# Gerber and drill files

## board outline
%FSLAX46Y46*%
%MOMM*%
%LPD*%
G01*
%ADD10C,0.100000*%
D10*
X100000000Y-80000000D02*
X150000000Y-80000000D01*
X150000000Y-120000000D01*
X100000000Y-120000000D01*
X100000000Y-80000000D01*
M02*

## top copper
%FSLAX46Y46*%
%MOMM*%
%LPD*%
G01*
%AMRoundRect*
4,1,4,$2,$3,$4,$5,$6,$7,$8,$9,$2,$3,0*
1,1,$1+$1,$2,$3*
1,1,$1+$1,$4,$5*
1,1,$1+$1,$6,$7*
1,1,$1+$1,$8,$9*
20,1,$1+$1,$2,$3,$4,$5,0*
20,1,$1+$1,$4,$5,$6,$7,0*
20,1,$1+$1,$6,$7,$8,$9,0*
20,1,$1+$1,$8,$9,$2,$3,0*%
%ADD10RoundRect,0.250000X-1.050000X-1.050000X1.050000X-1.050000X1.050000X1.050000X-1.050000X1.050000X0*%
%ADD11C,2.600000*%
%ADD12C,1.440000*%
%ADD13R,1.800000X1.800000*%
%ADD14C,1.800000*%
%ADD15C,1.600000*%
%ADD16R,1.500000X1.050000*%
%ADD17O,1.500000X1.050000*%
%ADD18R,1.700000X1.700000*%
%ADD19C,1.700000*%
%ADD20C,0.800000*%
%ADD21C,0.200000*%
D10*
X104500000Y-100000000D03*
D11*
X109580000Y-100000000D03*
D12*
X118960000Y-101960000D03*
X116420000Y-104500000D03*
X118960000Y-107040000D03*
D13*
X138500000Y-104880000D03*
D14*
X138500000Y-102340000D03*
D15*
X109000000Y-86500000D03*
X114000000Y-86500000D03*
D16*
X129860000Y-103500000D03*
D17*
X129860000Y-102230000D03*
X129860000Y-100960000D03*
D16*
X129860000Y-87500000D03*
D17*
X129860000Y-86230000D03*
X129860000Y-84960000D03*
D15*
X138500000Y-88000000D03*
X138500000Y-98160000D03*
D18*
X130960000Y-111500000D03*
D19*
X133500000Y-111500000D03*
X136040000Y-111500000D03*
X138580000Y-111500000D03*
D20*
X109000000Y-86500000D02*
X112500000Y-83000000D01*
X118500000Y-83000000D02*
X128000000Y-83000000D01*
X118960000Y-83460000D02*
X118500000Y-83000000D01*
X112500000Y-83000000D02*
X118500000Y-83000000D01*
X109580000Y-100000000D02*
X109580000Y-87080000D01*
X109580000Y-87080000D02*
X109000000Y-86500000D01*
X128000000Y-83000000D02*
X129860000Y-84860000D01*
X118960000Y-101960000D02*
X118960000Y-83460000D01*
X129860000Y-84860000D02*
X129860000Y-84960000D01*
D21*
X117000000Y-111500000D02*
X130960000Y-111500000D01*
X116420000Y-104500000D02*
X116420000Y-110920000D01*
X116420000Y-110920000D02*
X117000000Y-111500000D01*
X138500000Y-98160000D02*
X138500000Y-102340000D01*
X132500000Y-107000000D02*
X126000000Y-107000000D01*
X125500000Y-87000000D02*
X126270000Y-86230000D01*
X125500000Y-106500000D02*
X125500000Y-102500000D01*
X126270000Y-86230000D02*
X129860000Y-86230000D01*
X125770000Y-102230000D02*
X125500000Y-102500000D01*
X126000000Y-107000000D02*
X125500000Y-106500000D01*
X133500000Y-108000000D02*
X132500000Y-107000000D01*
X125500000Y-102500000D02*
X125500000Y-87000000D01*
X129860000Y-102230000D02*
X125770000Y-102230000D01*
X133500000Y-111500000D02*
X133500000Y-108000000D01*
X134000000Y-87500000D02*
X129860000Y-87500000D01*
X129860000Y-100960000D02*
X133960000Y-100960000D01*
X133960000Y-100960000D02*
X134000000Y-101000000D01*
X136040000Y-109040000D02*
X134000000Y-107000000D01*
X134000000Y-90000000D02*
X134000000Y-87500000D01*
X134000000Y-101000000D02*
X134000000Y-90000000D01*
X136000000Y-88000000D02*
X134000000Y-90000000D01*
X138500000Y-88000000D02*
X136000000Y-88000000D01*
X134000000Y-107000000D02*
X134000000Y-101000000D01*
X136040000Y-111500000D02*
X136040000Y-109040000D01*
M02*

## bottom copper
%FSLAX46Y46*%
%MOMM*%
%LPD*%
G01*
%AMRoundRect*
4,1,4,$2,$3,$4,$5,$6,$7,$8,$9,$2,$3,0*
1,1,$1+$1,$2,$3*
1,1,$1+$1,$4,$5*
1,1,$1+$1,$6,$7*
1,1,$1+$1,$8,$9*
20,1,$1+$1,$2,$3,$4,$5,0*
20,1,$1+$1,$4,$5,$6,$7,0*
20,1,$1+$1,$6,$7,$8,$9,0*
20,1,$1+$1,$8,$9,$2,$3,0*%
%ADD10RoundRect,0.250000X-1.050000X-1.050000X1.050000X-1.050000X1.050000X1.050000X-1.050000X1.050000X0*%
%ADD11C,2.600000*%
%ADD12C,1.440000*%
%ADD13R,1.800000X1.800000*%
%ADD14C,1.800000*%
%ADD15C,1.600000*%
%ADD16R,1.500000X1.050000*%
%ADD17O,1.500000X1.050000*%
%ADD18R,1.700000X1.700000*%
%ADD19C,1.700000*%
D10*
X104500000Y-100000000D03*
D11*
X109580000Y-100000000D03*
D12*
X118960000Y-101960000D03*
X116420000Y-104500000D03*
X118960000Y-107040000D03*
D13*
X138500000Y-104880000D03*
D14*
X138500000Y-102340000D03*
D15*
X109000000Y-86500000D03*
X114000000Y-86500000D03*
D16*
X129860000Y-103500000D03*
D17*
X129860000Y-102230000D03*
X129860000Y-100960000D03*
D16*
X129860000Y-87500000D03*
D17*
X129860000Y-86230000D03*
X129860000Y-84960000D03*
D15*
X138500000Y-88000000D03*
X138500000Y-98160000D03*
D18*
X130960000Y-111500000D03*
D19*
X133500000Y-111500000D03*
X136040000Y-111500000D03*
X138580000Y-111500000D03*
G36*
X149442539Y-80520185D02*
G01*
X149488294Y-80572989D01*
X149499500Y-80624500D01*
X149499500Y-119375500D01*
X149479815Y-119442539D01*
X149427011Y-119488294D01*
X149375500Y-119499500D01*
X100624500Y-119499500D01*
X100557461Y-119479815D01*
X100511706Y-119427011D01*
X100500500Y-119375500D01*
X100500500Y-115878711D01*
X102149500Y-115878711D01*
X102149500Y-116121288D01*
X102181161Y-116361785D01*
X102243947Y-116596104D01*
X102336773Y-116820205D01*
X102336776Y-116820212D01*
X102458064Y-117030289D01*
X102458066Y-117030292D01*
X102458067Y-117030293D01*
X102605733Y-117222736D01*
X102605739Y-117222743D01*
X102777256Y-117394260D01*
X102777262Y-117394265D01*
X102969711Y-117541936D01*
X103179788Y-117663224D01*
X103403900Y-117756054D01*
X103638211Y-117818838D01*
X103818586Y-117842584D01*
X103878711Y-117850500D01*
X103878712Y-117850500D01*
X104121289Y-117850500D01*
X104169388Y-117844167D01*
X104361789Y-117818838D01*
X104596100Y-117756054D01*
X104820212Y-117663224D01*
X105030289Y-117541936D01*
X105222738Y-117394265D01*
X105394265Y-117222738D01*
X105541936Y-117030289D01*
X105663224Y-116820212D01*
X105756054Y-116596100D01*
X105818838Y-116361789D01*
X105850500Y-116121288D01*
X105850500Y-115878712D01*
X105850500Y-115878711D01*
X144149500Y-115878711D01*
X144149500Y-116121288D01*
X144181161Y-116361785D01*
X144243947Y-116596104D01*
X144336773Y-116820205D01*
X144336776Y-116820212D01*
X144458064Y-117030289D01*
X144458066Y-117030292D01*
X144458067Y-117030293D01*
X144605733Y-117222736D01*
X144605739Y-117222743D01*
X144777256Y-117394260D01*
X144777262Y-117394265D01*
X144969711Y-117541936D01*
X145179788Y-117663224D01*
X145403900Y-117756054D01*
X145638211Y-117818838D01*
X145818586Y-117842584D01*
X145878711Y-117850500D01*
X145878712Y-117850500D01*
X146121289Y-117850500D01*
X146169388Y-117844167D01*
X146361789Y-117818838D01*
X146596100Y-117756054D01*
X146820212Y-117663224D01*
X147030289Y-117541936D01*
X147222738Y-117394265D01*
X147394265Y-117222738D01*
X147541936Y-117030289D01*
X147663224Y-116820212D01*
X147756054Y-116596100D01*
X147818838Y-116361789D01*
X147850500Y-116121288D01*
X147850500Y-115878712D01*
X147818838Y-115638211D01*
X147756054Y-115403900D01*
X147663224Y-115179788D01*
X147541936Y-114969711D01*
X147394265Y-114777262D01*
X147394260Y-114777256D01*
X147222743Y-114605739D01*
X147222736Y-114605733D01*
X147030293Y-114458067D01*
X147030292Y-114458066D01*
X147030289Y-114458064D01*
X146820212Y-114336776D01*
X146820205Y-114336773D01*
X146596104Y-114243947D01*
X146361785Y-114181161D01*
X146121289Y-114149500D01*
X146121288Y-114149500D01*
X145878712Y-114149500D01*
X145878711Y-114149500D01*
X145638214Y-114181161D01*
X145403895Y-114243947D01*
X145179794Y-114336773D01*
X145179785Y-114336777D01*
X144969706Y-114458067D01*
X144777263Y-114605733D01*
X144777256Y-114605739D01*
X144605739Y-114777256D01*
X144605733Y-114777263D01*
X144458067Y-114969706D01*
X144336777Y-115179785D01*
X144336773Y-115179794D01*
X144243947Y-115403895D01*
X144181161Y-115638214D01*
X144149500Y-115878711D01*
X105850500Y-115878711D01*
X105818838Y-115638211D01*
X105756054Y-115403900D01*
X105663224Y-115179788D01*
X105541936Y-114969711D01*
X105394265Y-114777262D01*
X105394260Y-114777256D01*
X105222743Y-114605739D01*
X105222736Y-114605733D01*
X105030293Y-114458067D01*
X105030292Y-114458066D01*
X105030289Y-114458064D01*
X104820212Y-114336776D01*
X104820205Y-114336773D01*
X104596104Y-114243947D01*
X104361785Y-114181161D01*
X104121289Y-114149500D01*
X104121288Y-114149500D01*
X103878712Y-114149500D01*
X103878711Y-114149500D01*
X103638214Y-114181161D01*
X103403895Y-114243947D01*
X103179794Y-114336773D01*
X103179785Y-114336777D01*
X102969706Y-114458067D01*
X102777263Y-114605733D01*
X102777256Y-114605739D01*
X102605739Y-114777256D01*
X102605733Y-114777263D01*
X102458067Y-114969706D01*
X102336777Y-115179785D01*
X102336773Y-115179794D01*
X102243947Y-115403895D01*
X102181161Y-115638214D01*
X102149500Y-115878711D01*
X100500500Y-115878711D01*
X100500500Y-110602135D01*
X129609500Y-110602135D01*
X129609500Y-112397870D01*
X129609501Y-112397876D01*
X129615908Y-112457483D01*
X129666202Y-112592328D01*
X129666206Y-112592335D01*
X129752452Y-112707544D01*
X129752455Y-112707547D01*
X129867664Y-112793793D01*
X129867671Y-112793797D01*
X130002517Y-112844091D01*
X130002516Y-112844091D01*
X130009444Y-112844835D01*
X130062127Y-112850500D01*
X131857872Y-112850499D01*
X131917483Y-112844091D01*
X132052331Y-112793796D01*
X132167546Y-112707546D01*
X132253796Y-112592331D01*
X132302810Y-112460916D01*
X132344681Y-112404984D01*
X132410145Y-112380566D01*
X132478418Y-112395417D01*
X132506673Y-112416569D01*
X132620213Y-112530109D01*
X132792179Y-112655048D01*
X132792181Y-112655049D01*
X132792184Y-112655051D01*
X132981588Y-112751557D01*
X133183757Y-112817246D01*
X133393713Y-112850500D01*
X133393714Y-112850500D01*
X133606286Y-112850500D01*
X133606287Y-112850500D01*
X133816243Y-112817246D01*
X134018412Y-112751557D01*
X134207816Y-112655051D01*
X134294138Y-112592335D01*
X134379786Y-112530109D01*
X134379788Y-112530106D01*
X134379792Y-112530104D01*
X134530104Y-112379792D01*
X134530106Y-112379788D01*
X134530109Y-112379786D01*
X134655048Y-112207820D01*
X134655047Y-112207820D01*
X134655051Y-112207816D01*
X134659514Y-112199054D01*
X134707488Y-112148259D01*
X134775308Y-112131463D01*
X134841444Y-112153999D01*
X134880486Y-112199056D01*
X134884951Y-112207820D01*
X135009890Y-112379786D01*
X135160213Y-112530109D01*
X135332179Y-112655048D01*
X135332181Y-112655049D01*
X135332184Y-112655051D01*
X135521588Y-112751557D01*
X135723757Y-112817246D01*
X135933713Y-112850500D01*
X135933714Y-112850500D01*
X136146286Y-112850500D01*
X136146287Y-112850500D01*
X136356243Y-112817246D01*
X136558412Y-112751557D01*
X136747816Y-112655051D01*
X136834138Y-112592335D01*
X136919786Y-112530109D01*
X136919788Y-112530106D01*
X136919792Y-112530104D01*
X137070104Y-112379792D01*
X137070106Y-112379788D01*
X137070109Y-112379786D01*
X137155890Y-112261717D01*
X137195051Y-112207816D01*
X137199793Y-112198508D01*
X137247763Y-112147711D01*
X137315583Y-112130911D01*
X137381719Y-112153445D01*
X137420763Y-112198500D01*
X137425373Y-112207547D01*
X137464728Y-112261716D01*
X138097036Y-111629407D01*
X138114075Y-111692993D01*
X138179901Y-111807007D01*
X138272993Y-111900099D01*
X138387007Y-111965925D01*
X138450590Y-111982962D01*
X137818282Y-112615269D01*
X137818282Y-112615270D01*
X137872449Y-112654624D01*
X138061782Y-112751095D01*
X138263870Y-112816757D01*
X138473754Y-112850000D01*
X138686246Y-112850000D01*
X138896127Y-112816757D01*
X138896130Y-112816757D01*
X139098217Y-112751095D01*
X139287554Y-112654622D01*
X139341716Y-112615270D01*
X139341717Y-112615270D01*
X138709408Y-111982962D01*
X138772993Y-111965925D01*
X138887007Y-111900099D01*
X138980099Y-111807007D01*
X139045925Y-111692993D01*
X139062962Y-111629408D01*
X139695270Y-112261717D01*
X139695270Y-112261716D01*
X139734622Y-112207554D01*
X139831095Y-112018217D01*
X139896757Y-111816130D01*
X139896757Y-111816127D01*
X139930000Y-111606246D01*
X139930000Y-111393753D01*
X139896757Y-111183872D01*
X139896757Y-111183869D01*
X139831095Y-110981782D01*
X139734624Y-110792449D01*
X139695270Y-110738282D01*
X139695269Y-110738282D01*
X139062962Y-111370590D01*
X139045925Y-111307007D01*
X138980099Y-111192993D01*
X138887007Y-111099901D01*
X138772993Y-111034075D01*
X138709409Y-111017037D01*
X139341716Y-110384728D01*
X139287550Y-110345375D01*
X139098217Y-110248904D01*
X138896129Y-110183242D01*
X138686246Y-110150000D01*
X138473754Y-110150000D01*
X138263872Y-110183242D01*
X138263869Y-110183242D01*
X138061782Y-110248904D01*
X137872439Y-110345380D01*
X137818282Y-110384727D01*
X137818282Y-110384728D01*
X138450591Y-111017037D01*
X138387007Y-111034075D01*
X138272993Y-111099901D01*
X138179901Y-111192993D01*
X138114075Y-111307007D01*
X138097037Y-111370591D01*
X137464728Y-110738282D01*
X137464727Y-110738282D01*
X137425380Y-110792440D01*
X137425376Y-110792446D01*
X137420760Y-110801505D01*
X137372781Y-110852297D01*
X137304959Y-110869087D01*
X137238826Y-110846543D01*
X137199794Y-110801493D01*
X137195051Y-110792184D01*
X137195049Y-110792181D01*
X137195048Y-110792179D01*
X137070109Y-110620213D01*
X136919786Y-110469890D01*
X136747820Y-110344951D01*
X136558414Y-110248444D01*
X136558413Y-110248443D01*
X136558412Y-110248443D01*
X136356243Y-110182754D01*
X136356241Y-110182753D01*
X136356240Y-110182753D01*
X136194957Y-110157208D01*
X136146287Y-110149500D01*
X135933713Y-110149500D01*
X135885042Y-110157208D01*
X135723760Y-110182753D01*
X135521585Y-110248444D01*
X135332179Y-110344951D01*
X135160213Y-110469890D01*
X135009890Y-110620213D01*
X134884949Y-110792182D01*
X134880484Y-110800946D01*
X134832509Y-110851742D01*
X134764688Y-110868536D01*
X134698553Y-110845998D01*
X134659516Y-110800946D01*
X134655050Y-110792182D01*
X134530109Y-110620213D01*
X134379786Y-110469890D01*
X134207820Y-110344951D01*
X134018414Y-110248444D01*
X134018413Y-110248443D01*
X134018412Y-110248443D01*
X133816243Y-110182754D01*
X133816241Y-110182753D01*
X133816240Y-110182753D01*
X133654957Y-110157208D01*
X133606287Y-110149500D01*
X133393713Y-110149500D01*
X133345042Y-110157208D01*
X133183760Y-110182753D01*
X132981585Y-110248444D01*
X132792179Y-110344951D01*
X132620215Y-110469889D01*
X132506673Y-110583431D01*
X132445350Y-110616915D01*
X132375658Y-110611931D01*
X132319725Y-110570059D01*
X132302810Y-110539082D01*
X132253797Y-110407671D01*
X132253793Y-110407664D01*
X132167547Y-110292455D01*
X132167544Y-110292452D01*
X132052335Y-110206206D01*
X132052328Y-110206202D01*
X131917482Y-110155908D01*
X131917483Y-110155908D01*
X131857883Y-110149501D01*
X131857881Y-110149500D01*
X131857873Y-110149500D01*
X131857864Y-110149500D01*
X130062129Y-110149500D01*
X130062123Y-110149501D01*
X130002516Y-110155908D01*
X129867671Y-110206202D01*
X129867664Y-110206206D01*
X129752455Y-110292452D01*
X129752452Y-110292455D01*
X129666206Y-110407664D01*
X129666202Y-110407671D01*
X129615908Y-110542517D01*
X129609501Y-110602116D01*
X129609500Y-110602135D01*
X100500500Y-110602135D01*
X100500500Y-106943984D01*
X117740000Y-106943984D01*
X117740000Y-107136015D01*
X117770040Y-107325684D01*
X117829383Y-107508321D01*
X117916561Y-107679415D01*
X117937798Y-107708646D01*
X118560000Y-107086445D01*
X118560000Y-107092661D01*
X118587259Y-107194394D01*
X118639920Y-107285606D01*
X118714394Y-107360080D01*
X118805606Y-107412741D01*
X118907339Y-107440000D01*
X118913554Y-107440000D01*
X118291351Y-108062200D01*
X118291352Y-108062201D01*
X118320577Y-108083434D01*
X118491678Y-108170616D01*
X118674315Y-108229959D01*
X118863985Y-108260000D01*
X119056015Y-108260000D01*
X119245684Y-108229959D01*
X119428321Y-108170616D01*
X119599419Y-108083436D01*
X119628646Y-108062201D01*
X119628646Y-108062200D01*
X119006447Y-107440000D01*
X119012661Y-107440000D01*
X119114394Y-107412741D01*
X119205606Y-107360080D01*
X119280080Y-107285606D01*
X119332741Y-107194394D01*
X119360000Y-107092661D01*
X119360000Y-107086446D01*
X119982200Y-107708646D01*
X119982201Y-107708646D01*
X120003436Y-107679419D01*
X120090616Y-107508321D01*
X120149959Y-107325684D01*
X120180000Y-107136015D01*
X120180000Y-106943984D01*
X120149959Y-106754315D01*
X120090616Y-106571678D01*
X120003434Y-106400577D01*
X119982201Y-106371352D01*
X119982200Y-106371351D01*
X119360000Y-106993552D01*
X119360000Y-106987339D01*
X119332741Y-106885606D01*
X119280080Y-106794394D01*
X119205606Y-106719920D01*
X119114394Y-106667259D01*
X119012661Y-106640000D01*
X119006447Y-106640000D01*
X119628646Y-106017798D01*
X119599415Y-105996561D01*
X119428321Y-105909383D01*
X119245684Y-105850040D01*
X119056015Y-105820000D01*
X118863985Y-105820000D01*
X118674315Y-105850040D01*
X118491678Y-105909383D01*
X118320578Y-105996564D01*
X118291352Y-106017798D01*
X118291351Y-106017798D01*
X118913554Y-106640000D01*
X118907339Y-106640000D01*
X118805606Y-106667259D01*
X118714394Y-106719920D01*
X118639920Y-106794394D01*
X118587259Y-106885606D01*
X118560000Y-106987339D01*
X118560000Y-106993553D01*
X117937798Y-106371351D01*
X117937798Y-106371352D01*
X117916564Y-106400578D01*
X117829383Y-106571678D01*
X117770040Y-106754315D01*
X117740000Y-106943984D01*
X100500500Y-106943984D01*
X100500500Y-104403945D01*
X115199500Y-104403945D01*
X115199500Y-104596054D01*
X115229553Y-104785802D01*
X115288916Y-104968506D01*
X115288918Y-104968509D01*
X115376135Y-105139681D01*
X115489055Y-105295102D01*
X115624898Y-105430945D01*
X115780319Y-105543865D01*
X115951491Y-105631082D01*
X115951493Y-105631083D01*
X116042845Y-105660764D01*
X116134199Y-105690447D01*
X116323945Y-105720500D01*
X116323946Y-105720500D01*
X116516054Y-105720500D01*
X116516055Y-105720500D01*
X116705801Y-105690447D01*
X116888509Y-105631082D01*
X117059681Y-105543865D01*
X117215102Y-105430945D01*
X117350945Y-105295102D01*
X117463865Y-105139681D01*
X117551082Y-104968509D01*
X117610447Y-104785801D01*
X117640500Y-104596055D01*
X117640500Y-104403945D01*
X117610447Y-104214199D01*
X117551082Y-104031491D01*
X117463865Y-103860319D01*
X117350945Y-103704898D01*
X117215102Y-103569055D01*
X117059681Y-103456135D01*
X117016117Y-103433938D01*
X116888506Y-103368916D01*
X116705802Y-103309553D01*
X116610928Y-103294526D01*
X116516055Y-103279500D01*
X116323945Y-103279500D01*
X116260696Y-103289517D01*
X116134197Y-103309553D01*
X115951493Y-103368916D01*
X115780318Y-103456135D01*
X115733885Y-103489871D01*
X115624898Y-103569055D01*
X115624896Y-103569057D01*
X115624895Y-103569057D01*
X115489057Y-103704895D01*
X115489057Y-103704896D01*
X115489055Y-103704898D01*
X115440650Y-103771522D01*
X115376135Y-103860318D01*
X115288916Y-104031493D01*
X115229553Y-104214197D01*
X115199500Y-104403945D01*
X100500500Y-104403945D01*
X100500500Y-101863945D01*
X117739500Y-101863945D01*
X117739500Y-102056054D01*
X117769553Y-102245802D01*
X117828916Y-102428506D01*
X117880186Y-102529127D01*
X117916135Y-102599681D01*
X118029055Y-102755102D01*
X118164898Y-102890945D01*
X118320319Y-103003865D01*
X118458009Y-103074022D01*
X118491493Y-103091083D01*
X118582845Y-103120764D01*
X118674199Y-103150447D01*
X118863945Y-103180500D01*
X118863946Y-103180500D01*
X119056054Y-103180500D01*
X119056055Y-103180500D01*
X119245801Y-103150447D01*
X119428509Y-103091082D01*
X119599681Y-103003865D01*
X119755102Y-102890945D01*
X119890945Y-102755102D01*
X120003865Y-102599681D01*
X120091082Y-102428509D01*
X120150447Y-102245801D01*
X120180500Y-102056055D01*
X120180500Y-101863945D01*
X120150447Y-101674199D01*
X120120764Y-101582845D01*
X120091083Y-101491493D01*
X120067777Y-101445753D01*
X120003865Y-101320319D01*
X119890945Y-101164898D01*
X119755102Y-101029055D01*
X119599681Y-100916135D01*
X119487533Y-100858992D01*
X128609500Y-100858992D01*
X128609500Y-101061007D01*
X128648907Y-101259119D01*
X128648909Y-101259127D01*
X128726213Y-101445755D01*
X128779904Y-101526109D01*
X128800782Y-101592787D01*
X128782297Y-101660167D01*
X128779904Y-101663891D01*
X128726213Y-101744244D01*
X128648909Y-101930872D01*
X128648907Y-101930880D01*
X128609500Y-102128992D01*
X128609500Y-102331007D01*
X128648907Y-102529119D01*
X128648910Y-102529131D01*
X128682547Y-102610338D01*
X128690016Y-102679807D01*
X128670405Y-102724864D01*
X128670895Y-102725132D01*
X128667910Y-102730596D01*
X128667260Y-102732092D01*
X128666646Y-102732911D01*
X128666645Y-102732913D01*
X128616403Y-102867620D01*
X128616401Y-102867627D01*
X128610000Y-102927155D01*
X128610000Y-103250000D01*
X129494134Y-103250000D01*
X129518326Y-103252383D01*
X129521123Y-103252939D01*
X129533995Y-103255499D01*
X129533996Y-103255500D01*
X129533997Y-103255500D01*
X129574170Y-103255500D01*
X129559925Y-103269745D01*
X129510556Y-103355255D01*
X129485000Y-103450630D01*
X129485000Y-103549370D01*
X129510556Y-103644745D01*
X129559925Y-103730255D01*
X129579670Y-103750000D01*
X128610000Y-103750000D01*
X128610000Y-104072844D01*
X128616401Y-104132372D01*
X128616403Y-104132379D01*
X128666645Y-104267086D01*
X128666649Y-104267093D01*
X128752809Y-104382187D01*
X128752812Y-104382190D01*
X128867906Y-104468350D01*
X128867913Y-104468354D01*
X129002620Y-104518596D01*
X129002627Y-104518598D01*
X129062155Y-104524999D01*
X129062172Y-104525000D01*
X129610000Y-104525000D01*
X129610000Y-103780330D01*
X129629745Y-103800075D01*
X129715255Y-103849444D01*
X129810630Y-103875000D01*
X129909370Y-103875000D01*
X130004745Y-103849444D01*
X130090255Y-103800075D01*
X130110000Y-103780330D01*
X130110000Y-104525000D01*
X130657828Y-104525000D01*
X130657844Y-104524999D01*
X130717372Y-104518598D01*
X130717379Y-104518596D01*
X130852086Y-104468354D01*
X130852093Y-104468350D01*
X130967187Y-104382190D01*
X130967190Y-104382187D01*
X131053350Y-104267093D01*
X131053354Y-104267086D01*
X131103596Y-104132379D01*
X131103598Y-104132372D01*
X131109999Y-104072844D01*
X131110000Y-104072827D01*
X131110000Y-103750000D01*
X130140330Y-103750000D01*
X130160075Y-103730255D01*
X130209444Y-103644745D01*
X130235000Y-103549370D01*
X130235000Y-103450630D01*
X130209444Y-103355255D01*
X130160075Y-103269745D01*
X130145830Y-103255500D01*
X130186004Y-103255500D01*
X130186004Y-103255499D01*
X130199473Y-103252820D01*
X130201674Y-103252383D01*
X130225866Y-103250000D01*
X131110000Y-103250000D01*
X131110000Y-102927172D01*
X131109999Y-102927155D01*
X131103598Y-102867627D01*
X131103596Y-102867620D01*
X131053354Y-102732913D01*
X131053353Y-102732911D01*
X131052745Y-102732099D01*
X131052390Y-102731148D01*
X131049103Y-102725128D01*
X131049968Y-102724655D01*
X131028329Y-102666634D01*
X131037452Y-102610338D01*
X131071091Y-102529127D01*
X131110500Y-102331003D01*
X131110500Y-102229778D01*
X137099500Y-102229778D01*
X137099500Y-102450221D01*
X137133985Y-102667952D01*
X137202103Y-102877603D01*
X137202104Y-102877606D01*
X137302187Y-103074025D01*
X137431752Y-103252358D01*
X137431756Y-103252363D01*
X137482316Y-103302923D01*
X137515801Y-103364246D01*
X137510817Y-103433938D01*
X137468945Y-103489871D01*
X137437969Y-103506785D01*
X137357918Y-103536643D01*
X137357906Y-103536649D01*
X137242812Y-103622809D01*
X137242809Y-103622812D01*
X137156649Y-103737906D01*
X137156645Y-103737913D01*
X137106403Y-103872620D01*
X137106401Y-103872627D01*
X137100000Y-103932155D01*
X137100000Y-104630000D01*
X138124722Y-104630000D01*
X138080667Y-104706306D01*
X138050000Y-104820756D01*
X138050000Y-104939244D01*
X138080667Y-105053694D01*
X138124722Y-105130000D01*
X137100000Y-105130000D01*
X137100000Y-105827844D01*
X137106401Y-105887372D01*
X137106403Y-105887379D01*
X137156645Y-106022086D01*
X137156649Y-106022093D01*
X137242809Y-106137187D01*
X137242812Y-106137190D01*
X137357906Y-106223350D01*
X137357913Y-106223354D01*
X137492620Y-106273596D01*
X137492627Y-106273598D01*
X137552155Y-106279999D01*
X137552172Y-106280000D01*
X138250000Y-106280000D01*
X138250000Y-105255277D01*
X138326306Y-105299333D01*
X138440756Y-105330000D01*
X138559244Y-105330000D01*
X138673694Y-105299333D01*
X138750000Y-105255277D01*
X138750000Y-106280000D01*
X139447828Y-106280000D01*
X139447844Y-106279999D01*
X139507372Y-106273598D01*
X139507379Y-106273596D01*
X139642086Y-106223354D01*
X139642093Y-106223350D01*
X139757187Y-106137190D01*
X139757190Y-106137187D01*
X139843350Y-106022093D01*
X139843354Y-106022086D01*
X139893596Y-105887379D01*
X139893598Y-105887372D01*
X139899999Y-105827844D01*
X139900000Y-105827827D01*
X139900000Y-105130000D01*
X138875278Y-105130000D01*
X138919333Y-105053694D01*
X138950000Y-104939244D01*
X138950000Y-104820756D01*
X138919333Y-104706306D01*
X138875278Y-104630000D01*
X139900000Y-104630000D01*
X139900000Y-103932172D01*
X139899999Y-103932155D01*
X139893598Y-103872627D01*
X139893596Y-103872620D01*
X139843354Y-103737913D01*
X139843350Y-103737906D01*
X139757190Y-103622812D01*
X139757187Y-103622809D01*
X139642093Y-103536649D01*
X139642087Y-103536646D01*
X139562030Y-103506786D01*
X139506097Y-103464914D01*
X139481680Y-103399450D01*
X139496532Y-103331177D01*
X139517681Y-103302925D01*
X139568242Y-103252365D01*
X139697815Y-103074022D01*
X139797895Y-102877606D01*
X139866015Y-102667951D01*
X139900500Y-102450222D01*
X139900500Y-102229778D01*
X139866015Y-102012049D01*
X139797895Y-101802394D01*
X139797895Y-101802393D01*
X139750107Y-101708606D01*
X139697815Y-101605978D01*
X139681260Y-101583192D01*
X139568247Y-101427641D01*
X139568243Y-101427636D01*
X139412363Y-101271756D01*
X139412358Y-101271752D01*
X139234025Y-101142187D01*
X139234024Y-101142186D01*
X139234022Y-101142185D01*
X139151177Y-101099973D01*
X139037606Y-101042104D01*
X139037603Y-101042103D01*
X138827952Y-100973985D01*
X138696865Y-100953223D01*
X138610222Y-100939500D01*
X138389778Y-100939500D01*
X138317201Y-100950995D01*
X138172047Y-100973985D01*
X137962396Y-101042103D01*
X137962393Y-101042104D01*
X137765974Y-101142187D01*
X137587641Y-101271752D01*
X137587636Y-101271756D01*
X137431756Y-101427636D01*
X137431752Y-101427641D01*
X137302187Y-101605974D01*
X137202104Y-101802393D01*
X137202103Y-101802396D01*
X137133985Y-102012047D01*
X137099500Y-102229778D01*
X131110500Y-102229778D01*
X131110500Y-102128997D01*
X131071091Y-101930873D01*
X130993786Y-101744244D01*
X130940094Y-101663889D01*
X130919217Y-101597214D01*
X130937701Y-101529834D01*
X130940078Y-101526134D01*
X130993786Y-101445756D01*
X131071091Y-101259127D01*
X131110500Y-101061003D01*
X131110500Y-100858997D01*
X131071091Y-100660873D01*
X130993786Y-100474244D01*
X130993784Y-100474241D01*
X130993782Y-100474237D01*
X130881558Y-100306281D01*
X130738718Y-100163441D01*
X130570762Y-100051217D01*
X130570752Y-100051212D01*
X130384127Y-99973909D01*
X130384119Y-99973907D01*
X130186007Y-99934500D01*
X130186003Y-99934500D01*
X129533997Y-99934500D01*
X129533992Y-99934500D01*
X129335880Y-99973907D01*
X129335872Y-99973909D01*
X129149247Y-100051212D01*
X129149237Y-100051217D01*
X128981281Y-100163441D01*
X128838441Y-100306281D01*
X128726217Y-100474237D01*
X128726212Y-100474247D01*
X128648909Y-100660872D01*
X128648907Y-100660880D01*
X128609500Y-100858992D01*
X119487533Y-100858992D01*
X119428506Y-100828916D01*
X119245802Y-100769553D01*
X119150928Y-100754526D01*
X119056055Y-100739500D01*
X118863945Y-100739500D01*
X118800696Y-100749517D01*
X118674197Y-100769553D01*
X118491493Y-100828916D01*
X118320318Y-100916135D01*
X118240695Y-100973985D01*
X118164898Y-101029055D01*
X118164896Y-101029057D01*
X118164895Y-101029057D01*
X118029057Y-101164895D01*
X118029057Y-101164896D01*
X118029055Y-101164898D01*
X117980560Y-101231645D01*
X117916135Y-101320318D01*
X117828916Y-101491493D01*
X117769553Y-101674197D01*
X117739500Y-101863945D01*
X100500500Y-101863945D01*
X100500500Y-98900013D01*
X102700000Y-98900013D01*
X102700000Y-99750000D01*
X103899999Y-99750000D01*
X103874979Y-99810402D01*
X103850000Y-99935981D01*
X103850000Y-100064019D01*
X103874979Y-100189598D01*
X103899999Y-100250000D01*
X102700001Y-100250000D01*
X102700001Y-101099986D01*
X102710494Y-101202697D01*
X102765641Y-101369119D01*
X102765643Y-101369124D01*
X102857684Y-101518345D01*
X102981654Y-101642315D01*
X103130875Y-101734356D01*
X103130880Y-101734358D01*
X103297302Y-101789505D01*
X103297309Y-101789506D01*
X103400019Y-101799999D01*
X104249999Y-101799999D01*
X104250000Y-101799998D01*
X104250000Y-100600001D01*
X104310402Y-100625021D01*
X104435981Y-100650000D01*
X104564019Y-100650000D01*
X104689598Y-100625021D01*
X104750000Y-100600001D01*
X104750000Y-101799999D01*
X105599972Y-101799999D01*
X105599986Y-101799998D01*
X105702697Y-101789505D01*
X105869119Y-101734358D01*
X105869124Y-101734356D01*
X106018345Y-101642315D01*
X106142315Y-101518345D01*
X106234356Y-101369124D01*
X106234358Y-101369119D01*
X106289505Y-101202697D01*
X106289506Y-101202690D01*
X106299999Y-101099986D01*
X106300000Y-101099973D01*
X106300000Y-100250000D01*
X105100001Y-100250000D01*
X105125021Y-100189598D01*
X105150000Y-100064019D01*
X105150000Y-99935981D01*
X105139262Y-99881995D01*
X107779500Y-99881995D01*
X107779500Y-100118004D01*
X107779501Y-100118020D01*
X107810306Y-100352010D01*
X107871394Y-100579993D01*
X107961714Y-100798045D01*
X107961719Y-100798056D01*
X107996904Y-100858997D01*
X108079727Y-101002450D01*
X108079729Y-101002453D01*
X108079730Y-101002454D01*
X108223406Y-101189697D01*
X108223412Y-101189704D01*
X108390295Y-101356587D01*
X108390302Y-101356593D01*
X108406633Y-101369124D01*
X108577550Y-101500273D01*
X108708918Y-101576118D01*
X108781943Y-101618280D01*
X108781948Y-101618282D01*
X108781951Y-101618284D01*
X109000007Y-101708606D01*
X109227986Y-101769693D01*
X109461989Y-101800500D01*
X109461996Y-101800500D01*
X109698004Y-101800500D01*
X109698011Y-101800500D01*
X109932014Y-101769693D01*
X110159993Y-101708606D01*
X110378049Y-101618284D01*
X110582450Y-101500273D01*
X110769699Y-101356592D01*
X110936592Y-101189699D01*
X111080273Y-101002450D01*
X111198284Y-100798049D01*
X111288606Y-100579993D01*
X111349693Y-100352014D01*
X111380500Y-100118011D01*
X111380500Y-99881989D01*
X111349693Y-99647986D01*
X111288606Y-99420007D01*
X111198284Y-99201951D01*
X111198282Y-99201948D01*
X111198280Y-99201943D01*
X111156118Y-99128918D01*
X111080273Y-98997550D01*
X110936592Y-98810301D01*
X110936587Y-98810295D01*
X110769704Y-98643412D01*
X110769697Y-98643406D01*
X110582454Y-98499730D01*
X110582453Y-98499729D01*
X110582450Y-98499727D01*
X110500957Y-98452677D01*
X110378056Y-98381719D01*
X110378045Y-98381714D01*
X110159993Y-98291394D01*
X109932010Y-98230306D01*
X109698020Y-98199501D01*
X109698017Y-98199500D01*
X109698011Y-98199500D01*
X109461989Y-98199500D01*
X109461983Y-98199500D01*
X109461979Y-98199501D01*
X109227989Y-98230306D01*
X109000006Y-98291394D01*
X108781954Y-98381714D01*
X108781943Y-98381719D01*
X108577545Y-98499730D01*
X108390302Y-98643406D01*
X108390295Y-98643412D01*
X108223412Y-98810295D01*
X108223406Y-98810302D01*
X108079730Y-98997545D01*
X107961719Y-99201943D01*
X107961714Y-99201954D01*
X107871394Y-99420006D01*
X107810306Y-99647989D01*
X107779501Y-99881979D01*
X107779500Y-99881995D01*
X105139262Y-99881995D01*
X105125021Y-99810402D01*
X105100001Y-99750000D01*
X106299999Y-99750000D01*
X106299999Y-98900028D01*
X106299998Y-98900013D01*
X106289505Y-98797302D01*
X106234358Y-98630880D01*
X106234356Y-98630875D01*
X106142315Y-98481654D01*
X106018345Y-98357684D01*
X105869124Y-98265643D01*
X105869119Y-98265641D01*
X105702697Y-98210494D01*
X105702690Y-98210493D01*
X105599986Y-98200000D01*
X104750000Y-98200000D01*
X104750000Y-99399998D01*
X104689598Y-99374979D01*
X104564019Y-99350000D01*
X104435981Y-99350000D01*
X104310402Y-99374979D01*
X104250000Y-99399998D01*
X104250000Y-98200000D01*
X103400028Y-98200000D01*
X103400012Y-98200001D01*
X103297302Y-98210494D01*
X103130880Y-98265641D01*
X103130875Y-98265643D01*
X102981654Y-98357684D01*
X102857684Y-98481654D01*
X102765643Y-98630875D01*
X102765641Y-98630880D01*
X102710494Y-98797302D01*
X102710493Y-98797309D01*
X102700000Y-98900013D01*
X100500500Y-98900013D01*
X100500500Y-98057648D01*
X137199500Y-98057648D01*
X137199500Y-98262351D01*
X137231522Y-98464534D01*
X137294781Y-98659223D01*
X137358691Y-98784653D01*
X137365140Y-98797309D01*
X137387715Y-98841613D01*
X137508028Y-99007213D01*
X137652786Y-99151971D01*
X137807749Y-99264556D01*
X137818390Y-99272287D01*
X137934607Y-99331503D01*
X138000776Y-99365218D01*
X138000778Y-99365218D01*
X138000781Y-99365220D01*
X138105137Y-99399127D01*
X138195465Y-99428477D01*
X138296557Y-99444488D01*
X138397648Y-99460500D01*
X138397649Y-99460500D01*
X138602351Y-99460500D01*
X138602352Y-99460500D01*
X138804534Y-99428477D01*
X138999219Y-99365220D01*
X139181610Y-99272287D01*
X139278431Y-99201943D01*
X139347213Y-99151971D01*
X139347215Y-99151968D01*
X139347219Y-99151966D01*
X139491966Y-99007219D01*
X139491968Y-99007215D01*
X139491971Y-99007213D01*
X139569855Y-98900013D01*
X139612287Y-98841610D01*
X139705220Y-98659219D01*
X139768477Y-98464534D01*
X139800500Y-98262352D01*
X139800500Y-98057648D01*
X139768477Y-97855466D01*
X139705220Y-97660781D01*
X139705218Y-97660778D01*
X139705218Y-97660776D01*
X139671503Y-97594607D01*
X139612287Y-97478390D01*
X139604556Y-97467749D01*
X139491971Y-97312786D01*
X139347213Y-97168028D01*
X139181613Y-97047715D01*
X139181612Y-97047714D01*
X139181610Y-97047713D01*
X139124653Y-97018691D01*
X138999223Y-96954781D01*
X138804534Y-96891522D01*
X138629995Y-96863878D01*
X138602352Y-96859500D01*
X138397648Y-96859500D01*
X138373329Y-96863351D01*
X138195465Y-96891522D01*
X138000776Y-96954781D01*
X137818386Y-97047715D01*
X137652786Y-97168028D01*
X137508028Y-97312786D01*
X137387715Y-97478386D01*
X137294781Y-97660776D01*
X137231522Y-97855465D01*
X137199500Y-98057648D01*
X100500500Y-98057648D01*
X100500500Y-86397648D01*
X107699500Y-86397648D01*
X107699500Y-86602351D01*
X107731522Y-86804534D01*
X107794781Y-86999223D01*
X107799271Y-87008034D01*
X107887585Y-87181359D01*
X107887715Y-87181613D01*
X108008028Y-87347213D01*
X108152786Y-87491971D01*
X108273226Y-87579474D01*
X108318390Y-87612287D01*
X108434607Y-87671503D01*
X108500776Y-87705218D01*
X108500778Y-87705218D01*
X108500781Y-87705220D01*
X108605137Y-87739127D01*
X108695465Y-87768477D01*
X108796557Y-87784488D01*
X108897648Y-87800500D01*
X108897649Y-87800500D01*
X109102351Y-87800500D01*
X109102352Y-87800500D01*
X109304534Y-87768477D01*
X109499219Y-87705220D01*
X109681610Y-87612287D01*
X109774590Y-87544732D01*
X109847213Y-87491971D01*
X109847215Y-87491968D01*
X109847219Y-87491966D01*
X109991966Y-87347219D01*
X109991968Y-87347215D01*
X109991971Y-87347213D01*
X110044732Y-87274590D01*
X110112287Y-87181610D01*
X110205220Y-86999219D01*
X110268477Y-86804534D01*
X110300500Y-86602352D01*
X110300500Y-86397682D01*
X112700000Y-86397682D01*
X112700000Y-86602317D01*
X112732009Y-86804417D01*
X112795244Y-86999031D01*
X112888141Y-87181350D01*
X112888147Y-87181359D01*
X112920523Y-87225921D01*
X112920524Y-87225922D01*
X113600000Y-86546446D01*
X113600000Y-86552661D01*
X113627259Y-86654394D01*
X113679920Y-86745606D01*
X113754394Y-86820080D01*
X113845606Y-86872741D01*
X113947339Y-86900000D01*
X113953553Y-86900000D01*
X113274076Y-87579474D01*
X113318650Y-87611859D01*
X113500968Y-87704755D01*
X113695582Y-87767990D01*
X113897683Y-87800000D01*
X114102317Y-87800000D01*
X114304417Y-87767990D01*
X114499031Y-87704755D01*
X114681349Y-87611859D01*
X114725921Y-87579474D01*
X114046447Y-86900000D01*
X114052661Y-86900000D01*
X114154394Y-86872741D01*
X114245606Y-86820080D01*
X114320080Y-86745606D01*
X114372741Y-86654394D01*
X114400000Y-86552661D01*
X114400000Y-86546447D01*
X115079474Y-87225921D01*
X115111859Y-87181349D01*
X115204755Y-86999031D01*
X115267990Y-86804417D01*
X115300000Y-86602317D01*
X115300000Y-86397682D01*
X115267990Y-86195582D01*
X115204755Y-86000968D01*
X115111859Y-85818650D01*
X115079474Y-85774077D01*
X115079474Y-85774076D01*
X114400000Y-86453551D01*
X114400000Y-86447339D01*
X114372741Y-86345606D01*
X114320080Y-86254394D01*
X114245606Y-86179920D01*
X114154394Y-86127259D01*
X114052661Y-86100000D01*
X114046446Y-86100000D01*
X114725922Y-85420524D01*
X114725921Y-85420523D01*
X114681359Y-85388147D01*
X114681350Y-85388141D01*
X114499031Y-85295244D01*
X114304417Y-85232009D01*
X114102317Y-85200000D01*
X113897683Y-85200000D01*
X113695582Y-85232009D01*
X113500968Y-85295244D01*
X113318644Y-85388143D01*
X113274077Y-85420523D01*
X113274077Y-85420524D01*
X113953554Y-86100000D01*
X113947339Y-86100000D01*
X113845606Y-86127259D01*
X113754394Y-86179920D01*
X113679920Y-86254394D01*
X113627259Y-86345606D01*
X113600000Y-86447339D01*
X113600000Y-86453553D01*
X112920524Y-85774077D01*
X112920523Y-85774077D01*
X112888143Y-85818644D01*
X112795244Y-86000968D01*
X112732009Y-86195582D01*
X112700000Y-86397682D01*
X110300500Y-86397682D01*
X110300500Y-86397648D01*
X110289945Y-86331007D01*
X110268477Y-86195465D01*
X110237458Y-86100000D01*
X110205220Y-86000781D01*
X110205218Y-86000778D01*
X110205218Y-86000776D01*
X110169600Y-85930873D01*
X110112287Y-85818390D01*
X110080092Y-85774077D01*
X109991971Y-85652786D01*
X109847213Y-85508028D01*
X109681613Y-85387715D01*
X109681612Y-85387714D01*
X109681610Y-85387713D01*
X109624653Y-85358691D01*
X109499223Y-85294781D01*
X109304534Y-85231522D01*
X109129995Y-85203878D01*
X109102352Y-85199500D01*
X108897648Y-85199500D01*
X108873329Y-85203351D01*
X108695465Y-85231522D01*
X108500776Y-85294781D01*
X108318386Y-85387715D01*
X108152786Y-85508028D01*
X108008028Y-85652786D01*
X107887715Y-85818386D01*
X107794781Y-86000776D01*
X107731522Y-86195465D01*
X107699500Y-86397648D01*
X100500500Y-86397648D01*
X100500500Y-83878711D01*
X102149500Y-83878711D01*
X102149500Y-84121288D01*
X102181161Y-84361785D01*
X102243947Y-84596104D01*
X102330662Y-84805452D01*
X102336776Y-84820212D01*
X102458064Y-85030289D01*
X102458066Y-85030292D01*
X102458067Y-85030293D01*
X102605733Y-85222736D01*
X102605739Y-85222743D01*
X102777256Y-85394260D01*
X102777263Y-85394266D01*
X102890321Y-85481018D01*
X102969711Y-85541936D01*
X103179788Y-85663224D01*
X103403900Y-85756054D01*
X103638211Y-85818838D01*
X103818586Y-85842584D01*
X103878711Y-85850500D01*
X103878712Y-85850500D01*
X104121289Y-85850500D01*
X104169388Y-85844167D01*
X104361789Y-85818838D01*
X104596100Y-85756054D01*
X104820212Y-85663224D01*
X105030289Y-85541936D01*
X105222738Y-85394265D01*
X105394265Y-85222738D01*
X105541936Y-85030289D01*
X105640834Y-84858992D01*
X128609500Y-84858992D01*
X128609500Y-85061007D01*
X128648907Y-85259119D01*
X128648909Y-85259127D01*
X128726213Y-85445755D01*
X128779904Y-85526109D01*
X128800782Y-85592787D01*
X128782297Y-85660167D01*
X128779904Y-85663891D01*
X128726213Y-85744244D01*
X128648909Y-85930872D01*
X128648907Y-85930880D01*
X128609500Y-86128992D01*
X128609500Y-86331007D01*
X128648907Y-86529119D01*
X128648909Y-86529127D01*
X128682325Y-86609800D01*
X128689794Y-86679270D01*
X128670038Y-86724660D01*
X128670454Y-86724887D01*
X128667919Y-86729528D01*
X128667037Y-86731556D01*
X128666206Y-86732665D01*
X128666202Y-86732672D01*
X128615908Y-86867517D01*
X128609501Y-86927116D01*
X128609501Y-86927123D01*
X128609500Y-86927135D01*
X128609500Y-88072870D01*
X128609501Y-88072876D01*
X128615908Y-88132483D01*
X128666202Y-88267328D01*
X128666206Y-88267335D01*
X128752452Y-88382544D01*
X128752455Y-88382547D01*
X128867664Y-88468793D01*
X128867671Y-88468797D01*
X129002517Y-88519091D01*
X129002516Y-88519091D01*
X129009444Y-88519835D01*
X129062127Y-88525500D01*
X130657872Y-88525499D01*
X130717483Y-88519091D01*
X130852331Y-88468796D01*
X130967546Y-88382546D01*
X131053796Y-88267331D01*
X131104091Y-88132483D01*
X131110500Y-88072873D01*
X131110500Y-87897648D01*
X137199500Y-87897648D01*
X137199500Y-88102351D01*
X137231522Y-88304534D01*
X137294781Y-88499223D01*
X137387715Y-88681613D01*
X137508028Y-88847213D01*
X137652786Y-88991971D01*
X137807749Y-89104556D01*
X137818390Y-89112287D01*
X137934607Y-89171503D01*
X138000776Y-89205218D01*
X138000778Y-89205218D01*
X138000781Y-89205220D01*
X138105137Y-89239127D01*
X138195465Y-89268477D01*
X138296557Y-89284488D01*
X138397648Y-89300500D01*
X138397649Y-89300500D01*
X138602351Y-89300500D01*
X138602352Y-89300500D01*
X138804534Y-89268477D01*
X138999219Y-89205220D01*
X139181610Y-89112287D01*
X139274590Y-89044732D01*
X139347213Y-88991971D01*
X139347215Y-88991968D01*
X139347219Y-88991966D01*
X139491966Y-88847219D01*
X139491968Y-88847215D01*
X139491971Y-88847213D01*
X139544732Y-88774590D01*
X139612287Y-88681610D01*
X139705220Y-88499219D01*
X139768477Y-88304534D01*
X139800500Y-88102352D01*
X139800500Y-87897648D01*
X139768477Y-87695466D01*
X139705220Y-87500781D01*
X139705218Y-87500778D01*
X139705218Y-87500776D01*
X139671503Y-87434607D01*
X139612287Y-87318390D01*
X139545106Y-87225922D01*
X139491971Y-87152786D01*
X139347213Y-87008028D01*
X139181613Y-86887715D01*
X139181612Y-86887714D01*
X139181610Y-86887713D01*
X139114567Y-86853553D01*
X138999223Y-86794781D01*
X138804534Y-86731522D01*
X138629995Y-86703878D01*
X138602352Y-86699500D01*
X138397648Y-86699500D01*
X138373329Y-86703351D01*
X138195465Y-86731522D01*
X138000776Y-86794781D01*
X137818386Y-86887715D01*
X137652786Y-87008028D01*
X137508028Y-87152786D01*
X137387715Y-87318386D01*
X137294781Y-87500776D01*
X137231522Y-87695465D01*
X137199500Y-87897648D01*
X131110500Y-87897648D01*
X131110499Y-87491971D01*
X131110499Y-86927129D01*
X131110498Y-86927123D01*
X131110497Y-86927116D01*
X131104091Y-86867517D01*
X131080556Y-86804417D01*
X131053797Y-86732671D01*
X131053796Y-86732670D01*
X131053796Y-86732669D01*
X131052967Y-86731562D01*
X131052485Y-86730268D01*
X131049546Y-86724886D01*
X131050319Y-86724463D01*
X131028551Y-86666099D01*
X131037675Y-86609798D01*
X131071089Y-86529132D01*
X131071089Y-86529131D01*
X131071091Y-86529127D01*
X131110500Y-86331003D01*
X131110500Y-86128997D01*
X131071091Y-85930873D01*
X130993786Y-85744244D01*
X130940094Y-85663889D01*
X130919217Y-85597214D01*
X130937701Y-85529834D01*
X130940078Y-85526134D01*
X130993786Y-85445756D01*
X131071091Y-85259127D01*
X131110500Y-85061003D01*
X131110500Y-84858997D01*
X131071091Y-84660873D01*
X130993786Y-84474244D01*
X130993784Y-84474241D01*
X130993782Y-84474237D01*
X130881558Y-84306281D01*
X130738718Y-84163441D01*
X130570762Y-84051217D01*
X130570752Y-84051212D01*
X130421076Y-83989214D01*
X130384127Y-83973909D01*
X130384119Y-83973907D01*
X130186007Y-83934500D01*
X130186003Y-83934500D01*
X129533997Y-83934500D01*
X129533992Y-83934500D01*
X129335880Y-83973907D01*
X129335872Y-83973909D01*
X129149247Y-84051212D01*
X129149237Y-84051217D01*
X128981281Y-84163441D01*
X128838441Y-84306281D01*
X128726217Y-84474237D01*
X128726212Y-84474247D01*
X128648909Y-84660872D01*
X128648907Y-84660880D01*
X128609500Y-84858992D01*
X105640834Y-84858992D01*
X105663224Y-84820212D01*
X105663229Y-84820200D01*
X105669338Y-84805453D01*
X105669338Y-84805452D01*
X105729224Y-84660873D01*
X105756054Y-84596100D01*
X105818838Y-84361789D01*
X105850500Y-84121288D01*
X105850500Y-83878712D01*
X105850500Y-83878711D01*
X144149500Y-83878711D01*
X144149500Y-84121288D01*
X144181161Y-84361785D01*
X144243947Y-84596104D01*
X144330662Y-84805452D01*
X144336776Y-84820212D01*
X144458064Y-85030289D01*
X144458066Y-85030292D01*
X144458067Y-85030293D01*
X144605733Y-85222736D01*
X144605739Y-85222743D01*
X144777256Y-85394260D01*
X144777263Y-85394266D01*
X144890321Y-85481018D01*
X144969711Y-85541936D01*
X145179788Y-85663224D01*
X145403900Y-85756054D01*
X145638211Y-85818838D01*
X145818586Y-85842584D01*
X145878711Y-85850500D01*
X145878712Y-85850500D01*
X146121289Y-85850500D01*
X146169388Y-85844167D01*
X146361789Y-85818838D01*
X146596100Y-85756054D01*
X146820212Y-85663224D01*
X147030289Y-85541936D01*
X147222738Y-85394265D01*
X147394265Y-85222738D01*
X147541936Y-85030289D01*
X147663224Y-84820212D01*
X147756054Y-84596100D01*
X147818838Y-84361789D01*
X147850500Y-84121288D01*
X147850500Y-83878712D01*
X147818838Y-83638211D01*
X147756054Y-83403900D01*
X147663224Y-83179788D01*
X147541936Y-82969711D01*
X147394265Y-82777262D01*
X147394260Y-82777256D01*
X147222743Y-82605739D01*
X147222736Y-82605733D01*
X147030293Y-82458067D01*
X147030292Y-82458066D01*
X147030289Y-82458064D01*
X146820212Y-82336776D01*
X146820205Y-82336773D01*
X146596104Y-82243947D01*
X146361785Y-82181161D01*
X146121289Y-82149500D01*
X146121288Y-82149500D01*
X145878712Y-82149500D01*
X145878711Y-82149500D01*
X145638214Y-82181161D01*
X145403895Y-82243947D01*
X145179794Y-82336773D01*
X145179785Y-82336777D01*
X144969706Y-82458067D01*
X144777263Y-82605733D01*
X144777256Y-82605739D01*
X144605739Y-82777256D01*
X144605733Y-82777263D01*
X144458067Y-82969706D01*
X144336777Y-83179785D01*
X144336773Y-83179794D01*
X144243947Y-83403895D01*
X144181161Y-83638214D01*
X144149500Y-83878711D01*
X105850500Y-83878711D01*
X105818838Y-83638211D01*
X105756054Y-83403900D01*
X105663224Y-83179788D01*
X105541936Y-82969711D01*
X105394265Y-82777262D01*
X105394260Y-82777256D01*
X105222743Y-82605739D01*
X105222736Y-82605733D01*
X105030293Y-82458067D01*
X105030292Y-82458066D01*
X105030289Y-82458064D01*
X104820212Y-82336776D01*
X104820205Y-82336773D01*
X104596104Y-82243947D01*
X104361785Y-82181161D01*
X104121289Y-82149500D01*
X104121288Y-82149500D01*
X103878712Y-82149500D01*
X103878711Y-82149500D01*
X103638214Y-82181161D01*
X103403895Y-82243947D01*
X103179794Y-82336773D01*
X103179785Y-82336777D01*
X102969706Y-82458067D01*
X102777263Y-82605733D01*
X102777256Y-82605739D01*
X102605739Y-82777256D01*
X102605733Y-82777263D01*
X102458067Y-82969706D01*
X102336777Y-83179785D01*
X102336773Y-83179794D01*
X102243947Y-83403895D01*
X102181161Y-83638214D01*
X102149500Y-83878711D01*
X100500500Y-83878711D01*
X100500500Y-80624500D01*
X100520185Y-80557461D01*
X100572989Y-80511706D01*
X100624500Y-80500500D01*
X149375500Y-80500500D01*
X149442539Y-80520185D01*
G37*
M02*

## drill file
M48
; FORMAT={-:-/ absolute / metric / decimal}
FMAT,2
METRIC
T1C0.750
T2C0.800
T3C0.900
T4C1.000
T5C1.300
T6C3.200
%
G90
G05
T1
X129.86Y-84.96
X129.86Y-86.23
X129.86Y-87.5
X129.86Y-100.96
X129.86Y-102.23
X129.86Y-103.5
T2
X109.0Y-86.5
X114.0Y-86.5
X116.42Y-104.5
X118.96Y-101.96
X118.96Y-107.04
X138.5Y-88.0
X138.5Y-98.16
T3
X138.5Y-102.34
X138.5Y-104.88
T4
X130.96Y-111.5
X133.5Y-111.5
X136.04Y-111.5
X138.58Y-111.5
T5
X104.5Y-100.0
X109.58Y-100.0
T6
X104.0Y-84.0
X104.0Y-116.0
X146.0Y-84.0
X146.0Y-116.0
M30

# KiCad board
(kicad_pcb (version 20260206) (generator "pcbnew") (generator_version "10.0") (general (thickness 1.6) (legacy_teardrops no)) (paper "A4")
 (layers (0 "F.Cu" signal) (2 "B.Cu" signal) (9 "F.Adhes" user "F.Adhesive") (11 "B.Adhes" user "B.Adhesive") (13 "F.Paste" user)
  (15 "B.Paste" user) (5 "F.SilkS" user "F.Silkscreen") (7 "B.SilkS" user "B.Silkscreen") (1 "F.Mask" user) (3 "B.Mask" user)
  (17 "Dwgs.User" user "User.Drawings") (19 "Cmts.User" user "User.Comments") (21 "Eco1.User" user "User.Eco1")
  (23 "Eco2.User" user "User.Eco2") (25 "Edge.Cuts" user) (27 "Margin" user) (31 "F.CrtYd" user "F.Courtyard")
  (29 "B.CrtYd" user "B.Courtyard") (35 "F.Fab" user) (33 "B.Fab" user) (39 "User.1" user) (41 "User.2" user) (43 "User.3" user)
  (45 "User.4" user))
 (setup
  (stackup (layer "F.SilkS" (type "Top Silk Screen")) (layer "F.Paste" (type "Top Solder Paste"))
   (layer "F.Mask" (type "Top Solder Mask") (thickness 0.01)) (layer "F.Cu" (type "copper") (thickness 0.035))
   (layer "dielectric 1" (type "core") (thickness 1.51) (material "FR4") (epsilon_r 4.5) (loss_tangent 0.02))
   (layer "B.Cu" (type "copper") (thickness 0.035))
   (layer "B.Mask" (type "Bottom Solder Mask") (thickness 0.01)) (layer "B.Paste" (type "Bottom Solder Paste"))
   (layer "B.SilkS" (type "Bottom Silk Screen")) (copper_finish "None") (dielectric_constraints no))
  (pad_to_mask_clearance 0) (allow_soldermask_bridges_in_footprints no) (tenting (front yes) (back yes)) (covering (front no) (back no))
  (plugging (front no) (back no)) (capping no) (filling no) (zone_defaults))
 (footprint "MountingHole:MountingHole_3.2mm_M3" (layer "F.Cu") (at 146 116)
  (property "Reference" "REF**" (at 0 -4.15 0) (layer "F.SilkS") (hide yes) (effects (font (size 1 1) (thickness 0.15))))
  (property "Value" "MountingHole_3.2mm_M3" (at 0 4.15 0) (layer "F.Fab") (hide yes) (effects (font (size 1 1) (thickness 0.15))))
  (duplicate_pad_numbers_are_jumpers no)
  (pad "" np_thru_hole circle (at 0 0) (size 3.2 3.2) (drill 3.2) (layers "*.Cu" "*.Mask")))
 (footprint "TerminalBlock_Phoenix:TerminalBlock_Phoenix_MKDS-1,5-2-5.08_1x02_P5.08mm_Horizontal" (layer "F.Cu") (at 104.5 100)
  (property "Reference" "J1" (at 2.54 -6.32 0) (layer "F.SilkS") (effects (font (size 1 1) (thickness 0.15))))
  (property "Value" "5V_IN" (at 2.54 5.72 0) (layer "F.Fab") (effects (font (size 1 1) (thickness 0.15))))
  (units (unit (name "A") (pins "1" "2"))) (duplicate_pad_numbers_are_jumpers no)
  (pad "1" thru_hole roundrect (at 0 0) (size 2.6 2.6) (drill 1.3) (layers "*.Cu" "*.Mask") (remove_unused_layers no)
   (roundrect_rratio 0.096154) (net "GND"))
  (pad "2" thru_hole circle (at 5.08 0) (size 2.6 2.6) (drill 1.3) (layers "*.Cu" "*.Mask") (remove_unused_layers no) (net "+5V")))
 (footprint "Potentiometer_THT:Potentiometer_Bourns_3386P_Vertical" (layer "F.Cu") (at 118.96 101.96 180)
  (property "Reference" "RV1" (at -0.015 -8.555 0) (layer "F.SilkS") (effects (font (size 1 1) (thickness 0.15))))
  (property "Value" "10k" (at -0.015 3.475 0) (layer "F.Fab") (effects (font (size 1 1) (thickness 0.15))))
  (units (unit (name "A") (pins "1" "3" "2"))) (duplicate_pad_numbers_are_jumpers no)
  (pad "1" thru_hole circle (at 0 0 180) (size 1.44 1.44) (drill 0.8) (layers "*.Cu" "*.Mask") (remove_unused_layers no) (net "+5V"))
  (pad "2" thru_hole circle (at 2.54 -2.54 180) (size 1.44 1.44) (drill 0.8) (layers "*.Cu" "*.Mask") (remove_unused_layers no)
   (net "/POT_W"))
  (pad "3" thru_hole circle (at 0 -5.08 180) (size 1.44 1.44) (drill 0.8) (layers "*.Cu" "*.Mask") (remove_unused_layers no) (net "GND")))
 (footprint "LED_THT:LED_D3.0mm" (layer "F.Cu") (at 138.5 104.88 90)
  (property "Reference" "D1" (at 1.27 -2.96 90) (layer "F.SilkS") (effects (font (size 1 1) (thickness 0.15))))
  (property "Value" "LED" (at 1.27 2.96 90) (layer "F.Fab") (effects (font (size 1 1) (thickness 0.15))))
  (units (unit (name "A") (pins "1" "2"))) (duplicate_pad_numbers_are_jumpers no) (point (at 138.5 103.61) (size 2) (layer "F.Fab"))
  (pad "1" thru_hole rect (at 0 0 90) (size 1.8 1.8) (drill 0.9) (layers "*.Cu" "*.Mask") (remove_unused_layers no) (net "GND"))
  (pad "2" thru_hole circle (at 2.54 0 90) (size 1.8 1.8) (drill 0.9) (layers "*.Cu" "*.Mask") (remove_unused_layers no) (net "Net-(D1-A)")))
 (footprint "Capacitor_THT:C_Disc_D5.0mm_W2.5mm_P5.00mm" (layer "F.Cu") (at 109 86.5)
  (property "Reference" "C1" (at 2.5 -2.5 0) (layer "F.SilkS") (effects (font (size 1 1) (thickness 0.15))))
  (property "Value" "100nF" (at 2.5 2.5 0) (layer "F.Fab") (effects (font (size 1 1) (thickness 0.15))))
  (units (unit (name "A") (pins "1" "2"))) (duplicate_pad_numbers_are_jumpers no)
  (pad "1" thru_hole circle (at 0 0) (size 1.6 1.6) (drill 0.8) (layers "*.Cu" "*.Mask") (remove_unused_layers no) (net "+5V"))
  (pad "2" thru_hole circle (at 5 0) (size 1.6 1.6) (drill 0.8) (layers "*.Cu" "*.Mask") (remove_unused_layers no) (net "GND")))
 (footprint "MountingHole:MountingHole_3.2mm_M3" (layer "F.Cu") (at 146 84)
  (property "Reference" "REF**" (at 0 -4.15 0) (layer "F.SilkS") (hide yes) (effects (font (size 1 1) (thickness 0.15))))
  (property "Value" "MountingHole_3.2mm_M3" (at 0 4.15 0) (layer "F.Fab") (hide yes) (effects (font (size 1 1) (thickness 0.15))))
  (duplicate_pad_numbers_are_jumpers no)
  (pad "" np_thru_hole circle (at 0 0) (size 3.2 3.2) (drill 3.2) (layers "*.Cu" "*.Mask")))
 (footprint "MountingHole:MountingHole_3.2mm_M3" (layer "F.Cu") (at 104 84)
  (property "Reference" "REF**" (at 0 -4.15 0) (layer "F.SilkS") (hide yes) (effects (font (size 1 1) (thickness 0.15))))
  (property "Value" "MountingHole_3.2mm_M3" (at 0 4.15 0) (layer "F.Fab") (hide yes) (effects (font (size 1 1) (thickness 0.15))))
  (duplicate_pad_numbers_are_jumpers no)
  (pad "" np_thru_hole circle (at 0 0) (size 3.2 3.2) (drill 3.2) (layers "*.Cu" "*.Mask")))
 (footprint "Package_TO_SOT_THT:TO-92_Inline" (layer "F.Cu") (at 129.86 103.5 90)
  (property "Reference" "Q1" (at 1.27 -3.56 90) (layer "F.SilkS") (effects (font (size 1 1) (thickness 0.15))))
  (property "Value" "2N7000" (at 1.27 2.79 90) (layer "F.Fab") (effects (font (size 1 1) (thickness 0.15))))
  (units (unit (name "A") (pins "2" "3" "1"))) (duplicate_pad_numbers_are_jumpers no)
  (pad "1" thru_hole rect (at 0 0 90) (size 1.05 1.5) (drill 0.75) (layers "*.Cu" "*.Mask") (remove_unused_layers no) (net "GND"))
  (pad "2" thru_hole oval (at 1.27 0 90) (size 1.05 1.5) (drill 0.75) (layers "*.Cu" "*.Mask") (remove_unused_layers no) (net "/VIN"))
  (pad "3" thru_hole oval (at 2.54 0 90) (size 1.05 1.5) (drill 0.75) (layers "*.Cu" "*.Mask") (remove_unused_layers no) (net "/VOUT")))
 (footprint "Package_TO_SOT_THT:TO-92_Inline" (layer "F.Cu") (at 129.86 87.5 90)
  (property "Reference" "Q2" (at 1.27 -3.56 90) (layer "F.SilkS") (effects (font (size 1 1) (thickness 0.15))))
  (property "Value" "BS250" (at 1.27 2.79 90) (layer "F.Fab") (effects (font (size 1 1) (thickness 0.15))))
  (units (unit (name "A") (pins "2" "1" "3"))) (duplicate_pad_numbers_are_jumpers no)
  (pad "1" thru_hole rect (at 0 0 90) (size 1.05 1.5) (drill 0.75) (layers "*.Cu" "*.Mask") (remove_unused_layers no) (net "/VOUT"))
  (pad "2" thru_hole oval (at 1.27 0 90) (size 1.05 1.5) (drill 0.75) (layers "*.Cu" "*.Mask") (remove_unused_layers no) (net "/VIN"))
  (pad "3" thru_hole oval (at 2.54 0 90) (size 1.05 1.5) (drill 0.75) (layers "*.Cu" "*.Mask") (remove_unused_layers no) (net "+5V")))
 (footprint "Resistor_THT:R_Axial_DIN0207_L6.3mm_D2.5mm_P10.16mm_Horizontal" (layer "F.Cu") (at 138.5 88 -90)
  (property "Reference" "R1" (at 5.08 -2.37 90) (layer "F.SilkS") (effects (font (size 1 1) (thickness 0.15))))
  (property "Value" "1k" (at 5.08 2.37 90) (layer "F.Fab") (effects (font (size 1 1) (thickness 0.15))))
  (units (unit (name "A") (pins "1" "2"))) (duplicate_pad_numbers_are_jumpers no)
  (pad "1" thru_hole circle (at 0 0 270) (size 1.6 1.6) (drill 0.8) (layers "*.Cu" "*.Mask") (remove_unused_layers no) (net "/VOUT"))
  (pad "2" thru_hole circle (at 10.16 0 270) (size 1.6 1.6) (drill 0.8) (layers "*.Cu" "*.Mask") (remove_unused_layers no)
   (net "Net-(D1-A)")))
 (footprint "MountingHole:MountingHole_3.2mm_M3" (layer "F.Cu") (at 104 116)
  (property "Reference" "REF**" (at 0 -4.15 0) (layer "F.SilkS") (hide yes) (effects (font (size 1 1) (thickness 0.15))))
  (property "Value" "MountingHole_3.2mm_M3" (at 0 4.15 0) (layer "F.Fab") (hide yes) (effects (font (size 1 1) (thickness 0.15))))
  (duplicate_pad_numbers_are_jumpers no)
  (pad "" np_thru_hole circle (at 0 0) (size 3.2 3.2) (drill 3.2) (layers "*.Cu" "*.Mask")))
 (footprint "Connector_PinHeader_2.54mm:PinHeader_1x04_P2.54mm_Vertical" (layer "F.Cu") (at 130.96 111.5 90)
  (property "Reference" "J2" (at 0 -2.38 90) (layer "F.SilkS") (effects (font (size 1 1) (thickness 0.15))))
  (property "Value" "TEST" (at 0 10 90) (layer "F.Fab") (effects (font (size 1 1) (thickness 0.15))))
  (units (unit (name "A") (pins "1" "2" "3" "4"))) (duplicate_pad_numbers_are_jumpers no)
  (pad "1" thru_hole rect (at 0 0 90) (size 1.7 1.7) (drill 1) (layers "*.Cu" "*.Mask") (remove_unused_layers no) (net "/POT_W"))
  (pad "2" thru_hole circle (at 0 2.54 90) (size 1.7 1.7) (drill 1) (layers "*.Cu" "*.Mask") (remove_unused_layers no) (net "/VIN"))
  (pad "3" thru_hole circle (at 0 5.08 90) (size 1.7 1.7) (drill 1) (layers "*.Cu" "*.Mask") (remove_unused_layers no) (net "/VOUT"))
  (pad "4" thru_hole circle (at 0 7.62 90) (size 1.7 1.7) (drill 1) (layers "*.Cu" "*.Mask") (remove_unused_layers no) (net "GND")))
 (gr_rect (start 100 80) (end 150 120) (stroke (width 0.1) (type solid)) (fill no) (layer "Edge.Cuts"))
 (segment (start 109 86.5) (end 112.5 83) (width 0.8) (layer "F.Cu") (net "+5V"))
 (segment (start 118.5 83) (end 128 83) (width 0.8) (layer "F.Cu") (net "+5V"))
 (segment (start 118.96 83.46) (end 118.5 83) (width 0.8) (layer "F.Cu") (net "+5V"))
 (segment (start 112.5 83) (end 118.5 83) (width 0.8) (layer "F.Cu") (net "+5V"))
 (segment (start 109.58 100) (end 109.58 87.08) (width 0.8) (layer "F.Cu") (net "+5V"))
 (segment (start 109.58 87.08) (end 109 86.5) (width 0.8) (layer "F.Cu") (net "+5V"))
 (segment (start 128 83) (end 129.86 84.86) (width 0.8) (layer "F.Cu") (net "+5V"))
 (segment (start 118.96 101.96) (end 118.96 83.46) (width 0.8) (layer "F.Cu") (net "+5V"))
 (segment (start 129.86 84.86) (end 129.86 84.96) (width 0.8) (layer "F.Cu") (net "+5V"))
 (segment (start 117 111.5) (end 130.96 111.5) (width 0.2) (layer "F.Cu") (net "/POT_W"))
 (segment (start 116.42 104.5) (end 116.42 110.92) (width 0.2) (layer "F.Cu") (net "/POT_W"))
 (segment (start 116.42 110.92) (end 117 111.5) (width 0.2) (layer "F.Cu") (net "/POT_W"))
 (segment (start 138.5 98.16) (end 138.5 102.34) (width 0.2) (layer "F.Cu") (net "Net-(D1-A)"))
 (segment (start 132.5 107) (end 126 107) (width 0.2) (layer "F.Cu") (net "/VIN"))
 (segment (start 125.5 87) (end 126.27 86.23) (width 0.2) (layer "F.Cu") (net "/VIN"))
 (segment (start 125.5 106.5) (end 125.5 102.5) (width 0.2) (layer "F.Cu") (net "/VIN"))
 (segment (start 126.27 86.23) (end 129.86 86.23) (width 0.2) (layer "F.Cu") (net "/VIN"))
 (segment (start 125.77 102.23) (end 125.5 102.5) (width 0.2) (layer "F.Cu") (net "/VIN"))
 (segment (start 126 107) (end 125.5 106.5) (width 0.2) (layer "F.Cu") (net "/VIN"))
 (segment (start 133.5 108) (end 132.5 107) (width 0.2) (layer "F.Cu") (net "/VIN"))
 (segment (start 125.5 102.5) (end 125.5 87) (width 0.2) (layer "F.Cu") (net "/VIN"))
 (segment (start 129.86 102.23) (end 125.77 102.23) (width 0.2) (layer "F.Cu") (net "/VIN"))
 (segment (start 133.5 111.5) (end 133.5 108) (width 0.2) (layer "F.Cu") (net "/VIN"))
 (segment (start 134 87.5) (end 129.86 87.5) (width 0.2) (layer "F.Cu") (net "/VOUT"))
 (segment (start 129.86 100.96) (end 133.96 100.96) (width 0.2) (layer "F.Cu") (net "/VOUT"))
 (segment (start 133.96 100.96) (end 134 101) (width 0.2) (layer "F.Cu") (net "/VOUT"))
 (segment (start 136.04 109.04) (end 134 107) (width 0.2) (layer "F.Cu") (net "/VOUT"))
 (segment (start 134 90) (end 134 87.5) (width 0.2) (layer "F.Cu") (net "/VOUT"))
 (segment (start 134 101) (end 134 90) (width 0.2) (layer "F.Cu") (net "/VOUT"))
 (segment (start 136 88) (end 134 90) (width 0.2) (layer "F.Cu") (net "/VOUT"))
 (segment (start 138.5 88) (end 136 88) (width 0.2) (layer "F.Cu") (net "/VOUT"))
 (segment (start 134 107) (end 134 101) (width 0.2) (layer "F.Cu") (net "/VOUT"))
 (segment (start 136.04 111.5) (end 136.04 109.04) (width 0.2) (layer "F.Cu") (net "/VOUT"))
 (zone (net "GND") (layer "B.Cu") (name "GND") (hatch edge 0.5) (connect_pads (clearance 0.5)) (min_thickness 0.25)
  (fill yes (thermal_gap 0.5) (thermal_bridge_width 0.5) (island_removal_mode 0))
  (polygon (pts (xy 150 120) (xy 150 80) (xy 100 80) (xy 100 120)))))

